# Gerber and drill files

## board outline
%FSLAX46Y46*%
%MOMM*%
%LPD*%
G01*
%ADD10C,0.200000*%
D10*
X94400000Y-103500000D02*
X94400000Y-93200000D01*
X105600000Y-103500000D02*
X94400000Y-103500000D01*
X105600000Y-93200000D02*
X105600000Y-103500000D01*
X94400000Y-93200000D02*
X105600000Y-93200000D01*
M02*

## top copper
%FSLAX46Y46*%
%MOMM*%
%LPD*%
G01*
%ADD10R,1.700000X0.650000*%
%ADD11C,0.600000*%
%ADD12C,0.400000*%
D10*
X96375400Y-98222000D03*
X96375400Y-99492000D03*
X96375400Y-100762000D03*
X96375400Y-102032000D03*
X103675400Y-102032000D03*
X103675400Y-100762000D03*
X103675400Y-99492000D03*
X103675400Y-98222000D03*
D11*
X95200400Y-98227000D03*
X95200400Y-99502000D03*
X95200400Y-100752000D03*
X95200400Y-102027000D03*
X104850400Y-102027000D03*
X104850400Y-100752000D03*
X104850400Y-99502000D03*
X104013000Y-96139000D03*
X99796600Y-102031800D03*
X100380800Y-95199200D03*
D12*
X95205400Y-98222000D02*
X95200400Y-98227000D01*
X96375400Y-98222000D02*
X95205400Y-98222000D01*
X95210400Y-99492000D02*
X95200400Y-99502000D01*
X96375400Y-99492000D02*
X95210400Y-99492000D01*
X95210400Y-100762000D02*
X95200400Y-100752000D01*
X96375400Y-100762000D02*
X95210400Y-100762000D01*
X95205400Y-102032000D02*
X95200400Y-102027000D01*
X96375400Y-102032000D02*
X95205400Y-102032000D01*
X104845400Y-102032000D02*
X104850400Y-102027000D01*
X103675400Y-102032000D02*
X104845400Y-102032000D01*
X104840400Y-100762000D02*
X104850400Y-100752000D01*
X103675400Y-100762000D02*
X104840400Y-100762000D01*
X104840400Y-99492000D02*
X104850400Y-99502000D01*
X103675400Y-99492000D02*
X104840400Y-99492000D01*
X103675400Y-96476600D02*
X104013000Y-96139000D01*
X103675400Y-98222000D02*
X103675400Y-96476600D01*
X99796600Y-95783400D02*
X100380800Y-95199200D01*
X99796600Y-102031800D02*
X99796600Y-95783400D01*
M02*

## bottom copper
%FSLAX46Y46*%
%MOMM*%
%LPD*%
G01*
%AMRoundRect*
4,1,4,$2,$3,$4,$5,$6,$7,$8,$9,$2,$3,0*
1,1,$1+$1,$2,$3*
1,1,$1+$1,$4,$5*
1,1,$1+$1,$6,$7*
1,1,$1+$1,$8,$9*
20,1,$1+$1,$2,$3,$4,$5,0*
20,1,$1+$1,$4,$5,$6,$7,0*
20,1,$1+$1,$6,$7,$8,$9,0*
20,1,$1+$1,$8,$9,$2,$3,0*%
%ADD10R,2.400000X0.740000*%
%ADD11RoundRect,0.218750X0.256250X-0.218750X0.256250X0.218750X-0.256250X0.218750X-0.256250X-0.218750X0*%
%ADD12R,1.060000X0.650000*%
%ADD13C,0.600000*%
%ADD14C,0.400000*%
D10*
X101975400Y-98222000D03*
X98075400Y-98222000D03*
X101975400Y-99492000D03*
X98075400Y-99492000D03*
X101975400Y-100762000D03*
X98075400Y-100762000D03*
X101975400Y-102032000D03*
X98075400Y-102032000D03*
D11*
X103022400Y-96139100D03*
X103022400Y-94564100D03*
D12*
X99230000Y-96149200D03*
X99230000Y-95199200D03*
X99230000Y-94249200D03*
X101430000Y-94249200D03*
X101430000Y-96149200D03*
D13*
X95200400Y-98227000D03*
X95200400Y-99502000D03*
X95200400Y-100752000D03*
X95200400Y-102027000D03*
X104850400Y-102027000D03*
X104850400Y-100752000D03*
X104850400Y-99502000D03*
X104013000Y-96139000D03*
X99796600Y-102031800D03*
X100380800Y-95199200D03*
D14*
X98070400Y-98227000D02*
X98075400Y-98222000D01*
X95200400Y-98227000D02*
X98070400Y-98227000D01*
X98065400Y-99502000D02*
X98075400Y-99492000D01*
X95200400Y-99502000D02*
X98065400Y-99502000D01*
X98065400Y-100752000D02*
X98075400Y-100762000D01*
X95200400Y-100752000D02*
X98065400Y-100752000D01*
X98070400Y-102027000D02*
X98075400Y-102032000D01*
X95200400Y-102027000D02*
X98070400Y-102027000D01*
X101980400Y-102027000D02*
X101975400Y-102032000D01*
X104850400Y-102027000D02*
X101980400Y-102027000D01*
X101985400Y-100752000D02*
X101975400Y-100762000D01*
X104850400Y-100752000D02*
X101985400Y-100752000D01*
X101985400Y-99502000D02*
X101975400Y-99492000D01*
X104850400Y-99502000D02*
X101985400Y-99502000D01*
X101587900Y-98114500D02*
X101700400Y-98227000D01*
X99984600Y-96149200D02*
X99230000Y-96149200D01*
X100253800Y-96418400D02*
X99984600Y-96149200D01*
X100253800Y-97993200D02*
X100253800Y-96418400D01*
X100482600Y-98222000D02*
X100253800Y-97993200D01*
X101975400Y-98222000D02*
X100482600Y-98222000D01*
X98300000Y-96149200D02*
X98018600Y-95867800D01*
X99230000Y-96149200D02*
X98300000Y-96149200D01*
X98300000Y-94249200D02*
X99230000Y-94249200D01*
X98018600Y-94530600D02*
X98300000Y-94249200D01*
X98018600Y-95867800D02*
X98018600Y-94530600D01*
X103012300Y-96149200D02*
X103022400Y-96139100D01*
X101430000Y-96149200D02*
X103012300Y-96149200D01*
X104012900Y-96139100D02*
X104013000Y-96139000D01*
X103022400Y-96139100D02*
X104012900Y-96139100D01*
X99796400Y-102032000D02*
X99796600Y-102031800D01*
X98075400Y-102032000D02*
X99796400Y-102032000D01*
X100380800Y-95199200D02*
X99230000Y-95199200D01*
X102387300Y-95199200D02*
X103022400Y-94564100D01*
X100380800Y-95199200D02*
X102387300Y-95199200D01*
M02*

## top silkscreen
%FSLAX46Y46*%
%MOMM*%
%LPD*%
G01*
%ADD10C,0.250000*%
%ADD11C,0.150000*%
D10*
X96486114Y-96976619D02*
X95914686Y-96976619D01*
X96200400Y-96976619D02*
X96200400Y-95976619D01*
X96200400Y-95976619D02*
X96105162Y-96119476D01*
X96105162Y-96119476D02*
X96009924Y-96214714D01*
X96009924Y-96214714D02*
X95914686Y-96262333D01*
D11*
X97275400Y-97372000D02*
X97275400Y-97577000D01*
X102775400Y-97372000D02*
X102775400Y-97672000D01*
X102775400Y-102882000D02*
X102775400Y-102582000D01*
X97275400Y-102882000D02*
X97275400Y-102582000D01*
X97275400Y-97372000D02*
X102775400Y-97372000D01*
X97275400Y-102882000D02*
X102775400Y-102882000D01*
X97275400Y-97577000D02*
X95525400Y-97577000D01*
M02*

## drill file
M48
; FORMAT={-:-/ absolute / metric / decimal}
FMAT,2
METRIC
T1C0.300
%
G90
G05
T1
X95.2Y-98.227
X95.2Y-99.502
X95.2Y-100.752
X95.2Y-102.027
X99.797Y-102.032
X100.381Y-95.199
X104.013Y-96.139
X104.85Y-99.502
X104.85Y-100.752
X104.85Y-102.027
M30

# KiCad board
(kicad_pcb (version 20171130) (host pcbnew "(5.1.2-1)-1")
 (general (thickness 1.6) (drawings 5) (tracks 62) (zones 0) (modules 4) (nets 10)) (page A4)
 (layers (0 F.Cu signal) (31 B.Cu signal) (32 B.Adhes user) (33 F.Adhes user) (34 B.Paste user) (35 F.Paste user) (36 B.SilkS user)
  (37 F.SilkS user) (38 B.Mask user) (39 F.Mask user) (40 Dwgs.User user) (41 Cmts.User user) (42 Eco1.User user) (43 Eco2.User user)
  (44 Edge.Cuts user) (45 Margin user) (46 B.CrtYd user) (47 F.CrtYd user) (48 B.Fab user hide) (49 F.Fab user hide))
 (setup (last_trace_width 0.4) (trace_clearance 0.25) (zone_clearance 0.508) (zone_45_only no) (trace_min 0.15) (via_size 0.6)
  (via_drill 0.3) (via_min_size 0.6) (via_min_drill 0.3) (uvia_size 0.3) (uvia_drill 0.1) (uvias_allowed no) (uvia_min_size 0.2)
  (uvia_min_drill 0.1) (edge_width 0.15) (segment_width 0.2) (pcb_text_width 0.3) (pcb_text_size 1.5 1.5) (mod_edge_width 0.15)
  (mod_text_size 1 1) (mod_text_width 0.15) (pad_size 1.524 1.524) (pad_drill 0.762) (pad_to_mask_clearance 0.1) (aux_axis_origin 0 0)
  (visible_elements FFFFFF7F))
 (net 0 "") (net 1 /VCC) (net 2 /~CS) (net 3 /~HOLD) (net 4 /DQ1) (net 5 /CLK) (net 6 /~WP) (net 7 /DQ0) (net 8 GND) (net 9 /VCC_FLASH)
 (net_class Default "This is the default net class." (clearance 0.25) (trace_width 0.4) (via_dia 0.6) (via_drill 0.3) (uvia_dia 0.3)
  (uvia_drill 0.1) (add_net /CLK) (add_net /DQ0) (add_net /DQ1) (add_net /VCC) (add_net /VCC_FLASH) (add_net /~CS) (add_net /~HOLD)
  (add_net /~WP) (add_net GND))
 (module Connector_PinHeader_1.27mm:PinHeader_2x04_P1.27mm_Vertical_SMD (layer B.Cu) (at 100.0254 100.127 180)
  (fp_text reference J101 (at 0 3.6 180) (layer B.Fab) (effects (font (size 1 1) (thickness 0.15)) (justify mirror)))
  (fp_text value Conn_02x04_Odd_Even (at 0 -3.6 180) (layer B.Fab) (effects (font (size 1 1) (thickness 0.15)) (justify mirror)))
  (pad 1 smd rect (at -1.95 1.905 180) (size 2.4 0.74) (layers B.Cu B.Paste B.Mask) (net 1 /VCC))
  (pad 2 smd rect (at 1.95 1.905 180) (size 2.4 0.74) (layers B.Cu B.Paste B.Mask) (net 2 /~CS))
  (pad 3 smd rect (at -1.95 0.635 180) (size 2.4 0.74) (layers B.Cu B.Paste B.Mask) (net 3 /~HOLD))
  (pad 4 smd rect (at 1.95 0.635 180) (size 2.4 0.74) (layers B.Cu B.Paste B.Mask) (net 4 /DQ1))
  (pad 5 smd rect (at -1.95 -0.635 180) (size 2.4 0.74) (layers B.Cu B.Paste B.Mask) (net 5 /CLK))
  (pad 6 smd rect (at 1.95 -0.635 180) (size 2.4 0.74) (layers B.Cu B.Paste B.Mask) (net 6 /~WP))
  (pad 7 smd rect (at -1.95 -1.905 180) (size 2.4 0.74) (layers B.Cu B.Paste B.Mask) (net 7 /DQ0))
  (pad 8 smd rect (at 1.95 -1.905 180) (size 2.4 0.74) (layers B.Cu B.Paste B.Mask) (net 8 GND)))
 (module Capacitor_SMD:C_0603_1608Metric (layer B.Cu) (at 103.0224 95.3516 90)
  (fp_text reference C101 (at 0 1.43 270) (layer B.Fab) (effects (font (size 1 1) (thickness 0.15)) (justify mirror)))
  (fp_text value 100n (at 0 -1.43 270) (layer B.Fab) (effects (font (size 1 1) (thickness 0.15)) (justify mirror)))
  (pad 1 smd roundrect (at -0.7875 0 90) (size 0.875 0.95) (layers B.Cu B.Paste B.Mask) (roundrect_rratio 0.25) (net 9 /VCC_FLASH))
  (pad 2 smd roundrect (at 0.7875 0 90) (size 0.875 0.95) (layers B.Cu B.Paste B.Mask) (roundrect_rratio 0.25) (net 8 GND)))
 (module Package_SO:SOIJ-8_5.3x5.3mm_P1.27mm (layer F.Cu) (at 100.0254 100.127)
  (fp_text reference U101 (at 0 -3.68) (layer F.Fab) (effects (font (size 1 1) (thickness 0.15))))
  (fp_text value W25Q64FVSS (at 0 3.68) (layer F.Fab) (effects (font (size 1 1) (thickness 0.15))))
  (fp_line (start -2.75 -2.755) (end -2.75 -2.55) (layer F.SilkS) (width 0.15))
  (fp_line (start 2.75 -2.755) (end 2.75 -2.455) (layer F.SilkS) (width 0.15))
  (fp_line (start 2.75 2.755) (end 2.75 2.455) (layer F.SilkS) (width 0.15))
  (fp_line (start -2.75 2.755) (end -2.75 2.455) (layer F.SilkS) (width 0.15))
  (fp_line (start -2.75 -2.755) (end 2.75 -2.755) (layer F.SilkS) (width 0.15))
  (fp_line (start -2.75 2.755) (end 2.75 2.755) (layer F.SilkS) (width 0.15))
  (fp_line (start -2.75 -2.55) (end -4.5 -2.55) (layer F.SilkS) (width 0.15))
  (pad 1 smd rect (at -3.65 -1.905) (size 1.7 0.65) (layers F.Cu F.Paste F.Mask) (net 2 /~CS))
  (pad 2 smd rect (at -3.65 -0.635) (size 1.7 0.65) (layers F.Cu F.Paste F.Mask) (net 4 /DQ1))
  (pad 3 smd rect (at -3.65 0.635) (size 1.7 0.65) (layers F.Cu F.Paste F.Mask) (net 6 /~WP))
  (pad 4 smd rect (at -3.65 1.905) (size 1.7 0.65) (layers F.Cu F.Paste F.Mask) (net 8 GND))
  (pad 5 smd rect (at 3.65 1.905) (size 1.7 0.65) (layers F.Cu F.Paste F.Mask) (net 7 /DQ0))
  (pad 6 smd rect (at 3.65 0.635) (size 1.7 0.65) (layers F.Cu F.Paste F.Mask) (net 5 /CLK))
  (pad 7 smd rect (at 3.65 -0.635) (size 1.7 0.65) (layers F.Cu F.Paste F.Mask) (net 3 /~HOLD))
  (pad 8 smd rect (at 3.65 -1.905) (size 1.7 0.65) (layers F.Cu F.Paste F.Mask) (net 9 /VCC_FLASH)))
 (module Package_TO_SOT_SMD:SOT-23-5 (layer B.Cu) (at 100.33 95.1992)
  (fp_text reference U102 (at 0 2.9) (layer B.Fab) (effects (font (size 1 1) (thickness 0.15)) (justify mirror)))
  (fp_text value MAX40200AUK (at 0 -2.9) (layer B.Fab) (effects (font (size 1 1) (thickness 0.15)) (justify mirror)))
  (pad 1 smd rect (at -1.1 0.95) (size 1.06 0.65) (layers B.Cu B.Paste B.Mask) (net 1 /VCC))
  (pad 2 smd rect (at -1.1 0) (size 1.06 0.65) (layers B.Cu B.Paste B.Mask) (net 8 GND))
  (pad 3 smd rect (at -1.1 -0.95) (size 1.06 0.65) (layers B.Cu B.Paste B.Mask) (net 1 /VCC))
  (pad 4 smd rect (at 1.1 -0.95) (size 1.06 0.65) (layers B.Cu B.Paste B.Mask))
  (pad 5 smd rect (at 1.1 0.95) (size 1.06 0.65) (layers B.Cu B.Paste B.Mask) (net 9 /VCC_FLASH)))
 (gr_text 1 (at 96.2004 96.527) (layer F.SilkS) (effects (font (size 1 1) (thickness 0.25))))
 (gr_line (start 94.4 103.5) (end 94.4 93.2) (layer Edge.Cuts) (width 0.2))
 (gr_line (start 105.6 103.5) (end 94.4 103.5) (layer Edge.Cuts) (width 0.2))
 (gr_line (start 105.6 93.2) (end 105.6 103.5) (layer Edge.Cuts) (width 0.2))
 (gr_line (start 94.4 93.2) (end 105.6 93.2) (layer Edge.Cuts) (width 0.2))
 (via (at 95.2004 98.227) (size 0.6) (drill 0.3) (layers F.Cu B.Cu) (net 2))
 (segment (start 95.2054 98.222) (end 95.2004 98.227) (width 0.4) (layer F.Cu) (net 2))
 (segment (start 96.3754 98.222) (end 95.2054 98.222) (width 0.4) (layer F.Cu) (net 2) (status 10))
 (segment (start 98.0704 98.227) (end 98.0754 98.222) (width 0.4) (layer B.Cu) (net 2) (status 30))
 (segment (start 95.2004 98.227) (end 98.0704 98.227) (width 0.4) (layer B.Cu) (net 2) (status 20))
 (via (at 95.2004 99.502) (size 0.6) (drill 0.3) (layers F.Cu B.Cu) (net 4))
 (segment (start 95.2104 99.492) (end 95.2004 99.502) (width 0.4) (layer F.Cu) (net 4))
 (segment (start 96.3754 99.492) (end 95.2104 99.492) (width 0.4) (layer F.Cu) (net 4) (status 10))
 (segment (start 98.0654 99.502) (end 98.0754 99.492) (width 0.4) (layer B.Cu) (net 4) (status 30))
 (segment (start 95.2004 99.502) (end 98.0654 99.502) (width 0.4) (layer B.Cu) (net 4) (status 20))
 (via (at 95.2004 100.752) (size 0.6) (drill 0.3) (layers F.Cu B.Cu) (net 6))
 (segment (start 95.2104 100.762) (end 95.2004 100.752) (width 0.4) (layer F.Cu) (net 6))
 (segment (start 96.3754 100.762) (end 95.2104 100.762) (width 0.4) (layer F.Cu) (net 6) (status 10))
 (segment (start 98.0654 100.752) (end 98.0754 100.762) (width 0.4) (layer B.Cu) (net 6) (status 30))
 (segment (start 95.2004 100.752) (end 98.0654 100.752) (width 0.4) (layer B.Cu) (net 6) (status 20))
 (via (at 95.2004 102.027) (size 0.6) (drill 0.3) (layers F.Cu B.Cu) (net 8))
 (segment (start 95.2054 102.032) (end 95.2004 102.027) (width 0.4) (layer F.Cu) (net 8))
 (segment (start 96.3754 102.032) (end 95.2054 102.032) (width 0.4) (layer F.Cu) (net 8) (status 10))
 (segment (start 98.0704 102.027) (end 98.0754 102.032) (width 0.4) (layer B.Cu) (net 8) (status 30))
 (segment (start 95.2004 102.027) (end 98.0704 102.027) (width 0.4) (layer B.Cu) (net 8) (status 20))
 (via (at 104.8504 102.027) (size 0.6) (drill 0.3) (layers F.Cu B.Cu) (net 7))
 (segment (start 104.8454 102.032) (end 104.8504 102.027) (width 0.4) (layer F.Cu) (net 7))
 (segment (start 103.6754 102.032) (end 104.8454 102.032) (width 0.4) (layer F.Cu) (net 7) (status 10))
 (segment (start 101.9804 102.027) (end 101.9754 102.032) (width 0.4) (layer B.Cu) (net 7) (status 30))
 (segment (start 104.8504 102.027) (end 101.9804 102.027) (width 0.4) (layer B.Cu) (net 7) (status 20))
 (segment (start 101.9854 100.752) (end 101.9754 100.762) (width 0.4) (layer B.Cu) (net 5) (status 30))
 (segment (start 104.8504 100.752) (end 101.9854 100.752) (width 0.4) (layer B.Cu) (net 5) (status 20))
 (via (at 104.8504 100.752) (size 0.6) (drill 0.3) (layers F.Cu B.Cu) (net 5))
 (segment (start 104.8404 100.762) (end 104.8504 100.752) (width 0.4) (layer F.Cu) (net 5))
 (segment (start 103.6754 100.762) (end 104.8404 100.762) (width 0.4) (layer F.Cu) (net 5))
 (segment (start 101.9854 99.502) (end 101.9754 99.492) (width 0.4) (layer B.Cu) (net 3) (status 30))
 (segment (start 104.8504 99.502) (end 101.9854 99.502) (width 0.4) (layer B.Cu) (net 3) (status 20))
 (via (at 104.8504 99.502) (size 0.6) (drill 0.3) (layers F.Cu B.Cu) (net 3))
 (segment (start 104.8404 99.492) (end 104.8504 99.502) (width 0.4) (layer F.Cu) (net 3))
 (segment (start 103.6754 99.492) (end 104.8404 99.492) (width 0.4) (layer F.Cu) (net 3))
 (segment (start 101.5879 98.1145) (end 101.7004 98.227) (width 0.4) (layer B.Cu) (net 1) (status 30))
 (segment (start 99.9846 96.1492) (end 99.23 96.1492) (width 0.4) (layer B.Cu) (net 1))
 (segment (start 100.2538 96.4184) (end 99.9846 96.1492) (width 0.4) (layer B.Cu) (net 1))
 (segment (start 100.2538 97.9932) (end 100.2538 96.4184) (width 0.4) (layer B.Cu) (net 1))
 (segment (start 100.4826 98.222) (end 100.2538 97.9932) (width 0.4) (layer B.Cu) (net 1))
 (segment (start 101.9754 98.222) (end 100.4826 98.222) (width 0.4) (layer B.Cu) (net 1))
 (segment (start 98.3 96.1492) (end 98.0186 95.8678) (width 0.4) (layer B.Cu) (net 1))
 (segment (start 99.23 96.1492) (end 98.3 96.1492) (width 0.4) (layer B.Cu) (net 1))
 (segment (start 98.3 94.2492) (end 99.23 94.2492) (width 0.4) (layer B.Cu) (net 1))
 (segment (start 98.0186 94.5306) (end 98.3 94.2492) (width 0.4) (layer B.Cu) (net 1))
 (segment (start 98.0186 95.8678) (end 98.0186 94.5306) (width 0.4) (layer B.Cu) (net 1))
 (segment (start 103.0123 96.1492) (end 103.0224 96.1391) (width 0.4) (layer B.Cu) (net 9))
 (segment (start 101.43 96.1492) (end 103.0123 96.1492) (width 0.4) (layer B.Cu) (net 9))
 (segment (start 104.0129 96.1391) (end 104.013 96.139) (width 0.4) (layer B.Cu) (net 9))
 (via (at 104.013 96.139) (size 0.6) (drill 0.3) (layers F.Cu B.Cu) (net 9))
 (segment (start 103.0224 96.1391) (end 104.0129 96.1391) (width 0.4) (layer B.Cu) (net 9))
 (segment (start 103.6754 96.4766) (end 104.013 96.139) (width 0.4) (layer F.Cu) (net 9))
 (segment (start 103.6754 98.222) (end 103.6754 96.4766) (width 0.4) (layer F.Cu) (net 9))
 (via (at 99.7966 102.0318) (size 0.6) (drill 0.3) (layers F.Cu B.Cu) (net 8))
 (segment (start 99.7964 102.032) (end 99.7966 102.0318) (width 0.4) (layer B.Cu) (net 8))
 (segment (start 98.0754 102.032) (end 99.7964 102.032) (width 0.4) (layer B.Cu) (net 8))
 (via (at 100.3808 95.1992) (size 0.6) (drill 0.3) (layers F.Cu B.Cu) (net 8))
 (segment (start 99.7966 95.7834) (end 100.3808 95.1992) (width 0.4) (layer F.Cu) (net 8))
 (segment (start 99.7966 102.0318) (end 99.7966 95.7834) (width 0.4) (layer F.Cu) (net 8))
 (segment (start 100.3808 95.1992) (end 99.23 95.1992) (width 0.4) (layer B.Cu) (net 8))
 (segment (start 102.3873 95.1992) (end 103.0224 94.5641) (width 0.4) (layer B.Cu) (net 8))
 (segment (start 100.3808 95.1992) (end 102.3873 95.1992) (width 0.4) (layer B.Cu) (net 8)))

